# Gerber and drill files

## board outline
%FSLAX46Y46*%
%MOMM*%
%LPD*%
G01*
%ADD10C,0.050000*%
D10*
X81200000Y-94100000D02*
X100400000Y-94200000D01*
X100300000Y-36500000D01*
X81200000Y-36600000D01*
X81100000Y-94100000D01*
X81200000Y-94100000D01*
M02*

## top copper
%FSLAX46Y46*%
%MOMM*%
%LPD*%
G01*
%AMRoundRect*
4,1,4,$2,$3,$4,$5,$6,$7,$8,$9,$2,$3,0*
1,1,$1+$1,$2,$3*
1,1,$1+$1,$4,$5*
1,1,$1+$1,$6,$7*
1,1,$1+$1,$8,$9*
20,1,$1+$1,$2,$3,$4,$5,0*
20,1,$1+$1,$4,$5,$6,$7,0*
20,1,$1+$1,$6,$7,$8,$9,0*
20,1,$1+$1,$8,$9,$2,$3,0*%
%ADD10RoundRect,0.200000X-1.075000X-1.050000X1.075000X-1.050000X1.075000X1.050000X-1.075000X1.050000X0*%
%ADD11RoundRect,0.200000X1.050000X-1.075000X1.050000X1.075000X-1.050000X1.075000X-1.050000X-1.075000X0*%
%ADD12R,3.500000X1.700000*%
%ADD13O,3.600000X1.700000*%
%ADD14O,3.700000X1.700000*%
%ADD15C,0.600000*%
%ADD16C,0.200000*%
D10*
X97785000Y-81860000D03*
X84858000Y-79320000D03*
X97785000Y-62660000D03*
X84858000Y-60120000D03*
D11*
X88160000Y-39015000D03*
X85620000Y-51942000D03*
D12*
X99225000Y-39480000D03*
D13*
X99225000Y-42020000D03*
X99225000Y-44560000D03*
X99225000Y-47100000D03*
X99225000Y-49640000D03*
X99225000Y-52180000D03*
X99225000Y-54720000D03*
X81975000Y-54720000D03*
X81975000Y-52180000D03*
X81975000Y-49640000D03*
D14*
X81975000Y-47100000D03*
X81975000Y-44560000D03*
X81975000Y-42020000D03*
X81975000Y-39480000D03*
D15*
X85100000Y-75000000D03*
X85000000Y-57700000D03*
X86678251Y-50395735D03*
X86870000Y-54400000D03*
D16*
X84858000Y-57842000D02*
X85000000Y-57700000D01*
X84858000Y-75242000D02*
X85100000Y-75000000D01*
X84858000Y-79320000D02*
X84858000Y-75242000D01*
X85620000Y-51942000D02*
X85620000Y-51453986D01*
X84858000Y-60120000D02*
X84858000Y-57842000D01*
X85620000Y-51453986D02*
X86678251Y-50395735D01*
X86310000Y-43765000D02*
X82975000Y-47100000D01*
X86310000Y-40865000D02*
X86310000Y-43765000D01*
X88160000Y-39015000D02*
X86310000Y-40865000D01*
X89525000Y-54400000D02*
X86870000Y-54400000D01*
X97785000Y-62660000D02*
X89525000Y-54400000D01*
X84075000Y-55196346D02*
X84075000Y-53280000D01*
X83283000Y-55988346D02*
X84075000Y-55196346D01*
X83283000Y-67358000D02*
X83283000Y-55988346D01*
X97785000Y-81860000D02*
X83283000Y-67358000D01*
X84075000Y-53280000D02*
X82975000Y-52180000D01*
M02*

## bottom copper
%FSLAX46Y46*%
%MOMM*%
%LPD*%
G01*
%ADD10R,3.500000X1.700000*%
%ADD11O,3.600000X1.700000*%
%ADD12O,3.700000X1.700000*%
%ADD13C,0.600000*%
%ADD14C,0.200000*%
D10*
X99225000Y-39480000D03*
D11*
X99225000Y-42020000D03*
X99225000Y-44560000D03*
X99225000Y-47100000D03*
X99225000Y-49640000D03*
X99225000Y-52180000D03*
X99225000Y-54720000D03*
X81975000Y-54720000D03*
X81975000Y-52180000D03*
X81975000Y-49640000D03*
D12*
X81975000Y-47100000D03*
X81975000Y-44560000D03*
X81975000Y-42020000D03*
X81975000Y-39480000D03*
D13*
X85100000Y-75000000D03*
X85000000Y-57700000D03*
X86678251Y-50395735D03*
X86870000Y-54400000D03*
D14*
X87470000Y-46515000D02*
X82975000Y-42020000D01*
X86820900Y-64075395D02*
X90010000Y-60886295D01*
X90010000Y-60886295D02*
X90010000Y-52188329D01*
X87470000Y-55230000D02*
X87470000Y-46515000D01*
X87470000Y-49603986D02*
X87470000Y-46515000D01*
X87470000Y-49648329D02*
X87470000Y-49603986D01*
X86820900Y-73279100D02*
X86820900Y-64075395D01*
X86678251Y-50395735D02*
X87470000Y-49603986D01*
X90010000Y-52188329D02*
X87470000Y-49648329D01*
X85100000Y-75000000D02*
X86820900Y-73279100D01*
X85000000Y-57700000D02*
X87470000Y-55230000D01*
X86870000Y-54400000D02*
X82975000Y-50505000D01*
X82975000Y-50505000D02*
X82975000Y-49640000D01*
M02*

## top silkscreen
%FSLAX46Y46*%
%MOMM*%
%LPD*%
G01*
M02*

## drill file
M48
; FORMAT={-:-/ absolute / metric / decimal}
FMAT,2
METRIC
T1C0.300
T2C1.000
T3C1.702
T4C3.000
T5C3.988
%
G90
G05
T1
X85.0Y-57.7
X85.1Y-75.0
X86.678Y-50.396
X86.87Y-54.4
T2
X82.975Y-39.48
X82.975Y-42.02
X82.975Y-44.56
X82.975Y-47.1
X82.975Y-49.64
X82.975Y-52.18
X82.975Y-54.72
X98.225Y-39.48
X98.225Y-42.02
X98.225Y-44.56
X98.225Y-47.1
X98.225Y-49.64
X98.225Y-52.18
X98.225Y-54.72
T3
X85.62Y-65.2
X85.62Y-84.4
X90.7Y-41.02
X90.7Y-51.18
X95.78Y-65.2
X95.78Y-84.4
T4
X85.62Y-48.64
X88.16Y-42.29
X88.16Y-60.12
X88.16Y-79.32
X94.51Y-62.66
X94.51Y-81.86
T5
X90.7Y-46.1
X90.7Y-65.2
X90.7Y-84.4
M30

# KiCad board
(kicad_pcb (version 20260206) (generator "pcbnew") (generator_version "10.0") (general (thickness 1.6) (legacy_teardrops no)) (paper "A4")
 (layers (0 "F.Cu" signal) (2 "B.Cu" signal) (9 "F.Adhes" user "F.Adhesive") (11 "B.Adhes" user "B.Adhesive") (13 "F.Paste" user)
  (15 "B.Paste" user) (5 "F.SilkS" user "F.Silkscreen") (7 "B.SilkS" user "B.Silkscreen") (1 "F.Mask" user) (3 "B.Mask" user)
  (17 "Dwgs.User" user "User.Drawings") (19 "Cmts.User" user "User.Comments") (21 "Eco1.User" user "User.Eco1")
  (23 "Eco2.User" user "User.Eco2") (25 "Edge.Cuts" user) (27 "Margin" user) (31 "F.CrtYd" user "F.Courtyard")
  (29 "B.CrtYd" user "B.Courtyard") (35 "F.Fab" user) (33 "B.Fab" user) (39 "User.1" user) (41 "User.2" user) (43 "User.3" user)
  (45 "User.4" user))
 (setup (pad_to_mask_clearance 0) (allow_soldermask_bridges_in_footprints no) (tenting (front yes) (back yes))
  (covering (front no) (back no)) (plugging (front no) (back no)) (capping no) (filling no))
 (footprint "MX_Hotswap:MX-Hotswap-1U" (layer "F.Cu") (at 90.7 84.4)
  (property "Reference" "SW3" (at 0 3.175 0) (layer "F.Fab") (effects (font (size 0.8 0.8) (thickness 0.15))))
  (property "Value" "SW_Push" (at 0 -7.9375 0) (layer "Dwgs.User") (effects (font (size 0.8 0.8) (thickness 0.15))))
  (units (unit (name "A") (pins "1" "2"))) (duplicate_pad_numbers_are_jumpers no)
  (pad "" np_thru_hole circle (at -5.08 0 311.901) (size 1.7018 1.7018) (drill 1.7018) (layers "*.Cu" "*.Mask"))
  (pad "" np_thru_hole circle (at -2.54 -5.08) (size 3 3) (drill 3) (layers "*.Cu" "*.Mask"))
  (pad "" np_thru_hole circle (at 0 0) (size 3.9878 3.9878) (drill 3.9878) (layers "*.Cu" "*.Mask"))
  (pad "" np_thru_hole circle (at 3.81 -2.54) (size 3 3) (drill 3) (layers "*.Cu" "*.Mask"))
  (pad "" np_thru_hole circle (at 5.08 0 311.901) (size 1.7018 1.7018) (drill 1.7018) (layers "*.Cu" "*.Mask"))
  (pad "1" smd roundrect (at 7.085 -2.54) (size 2.55 2.5) (layers "F.Cu" "F.Mask" "F.Paste") (roundrect_rratio 0.08)
   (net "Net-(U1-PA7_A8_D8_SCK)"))
  (pad "2" smd roundrect (at -5.842 -5.08) (size 2.55 2.5) (layers "F.Cu" "F.Mask" "F.Paste") (roundrect_rratio 0.08) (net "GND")))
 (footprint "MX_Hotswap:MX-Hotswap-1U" (layer "F.Cu") (at 90.7 65.2)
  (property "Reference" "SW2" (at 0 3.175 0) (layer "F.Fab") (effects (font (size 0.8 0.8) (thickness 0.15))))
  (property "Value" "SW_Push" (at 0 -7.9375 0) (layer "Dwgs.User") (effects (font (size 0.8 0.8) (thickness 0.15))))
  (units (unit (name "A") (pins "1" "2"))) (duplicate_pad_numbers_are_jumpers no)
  (pad "" np_thru_hole circle (at -5.08 0 311.901) (size 1.7018 1.7018) (drill 1.7018) (layers "*.Cu" "*.Mask"))
  (pad "" np_thru_hole circle (at -2.54 -5.08) (size 3 3) (drill 3) (layers "*.Cu" "*.Mask"))
  (pad "" np_thru_hole circle (at 0 0) (size 3.9878 3.9878) (drill 3.9878) (layers "*.Cu" "*.Mask"))
  (pad "" np_thru_hole circle (at 3.81 -2.54) (size 3 3) (drill 3) (layers "*.Cu" "*.Mask"))
  (pad "" np_thru_hole circle (at 5.08 0 311.901) (size 1.7018 1.7018) (drill 1.7018) (layers "*.Cu" "*.Mask"))
  (pad "1" smd roundrect (at 7.085 -2.54) (size 2.55 2.5) (layers "F.Cu" "F.Mask" "F.Paste") (roundrect_rratio 0.08)
   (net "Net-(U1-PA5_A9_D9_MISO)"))
  (pad "2" smd roundrect (at -5.842 -5.08) (size 2.55 2.5) (layers "F.Cu" "F.Mask" "F.Paste") (roundrect_rratio 0.08) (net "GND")))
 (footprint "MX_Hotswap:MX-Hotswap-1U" (layer "F.Cu") (at 90.7 46.1 90)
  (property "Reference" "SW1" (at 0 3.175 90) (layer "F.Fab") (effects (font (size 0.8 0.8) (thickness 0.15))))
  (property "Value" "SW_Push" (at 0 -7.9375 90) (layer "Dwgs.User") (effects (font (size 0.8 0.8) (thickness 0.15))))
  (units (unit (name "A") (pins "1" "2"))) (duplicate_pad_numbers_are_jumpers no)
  (pad "" np_thru_hole circle (at -5.08 0 41.901) (size 1.7018 1.7018) (drill 1.7018) (layers "*.Cu" "*.Mask"))
  (pad "" np_thru_hole circle (at -2.54 -5.08 90) (size 3 3) (drill 3) (layers "*.Cu" "*.Mask"))
  (pad "" np_thru_hole circle (at 0 0 90) (size 3.9878 3.9878) (drill 3.9878) (layers "*.Cu" "*.Mask"))
  (pad "" np_thru_hole circle (at 3.81 -2.54 90) (size 3 3) (drill 3) (layers "*.Cu" "*.Mask"))
  (pad "" np_thru_hole circle (at 5.08 0 41.901) (size 1.7018 1.7018) (drill 1.7018) (layers "*.Cu" "*.Mask"))
  (pad "1" smd roundrect (at 7.085 -2.54 90) (size 2.55 2.5) (layers "F.Cu" "F.Mask" "F.Paste") (roundrect_rratio 0.08)
   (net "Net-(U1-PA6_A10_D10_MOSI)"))
  (pad "2" smd roundrect (at -5.842 -5.08 90) (size 2.55 2.5) (layers "F.Cu" "F.Mask" "F.Paste") (roundrect_rratio 0.08) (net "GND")))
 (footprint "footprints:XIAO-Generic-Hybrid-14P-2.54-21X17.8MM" (layer "B.Cu") (at 90.6 47.1 180)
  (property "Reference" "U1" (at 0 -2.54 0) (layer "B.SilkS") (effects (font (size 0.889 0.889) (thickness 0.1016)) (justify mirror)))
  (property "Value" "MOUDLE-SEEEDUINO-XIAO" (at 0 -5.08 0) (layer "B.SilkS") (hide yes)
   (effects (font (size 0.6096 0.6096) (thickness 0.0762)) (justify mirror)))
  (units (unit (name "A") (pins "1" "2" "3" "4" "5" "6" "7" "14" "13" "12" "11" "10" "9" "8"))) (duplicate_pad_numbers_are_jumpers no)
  (pad "1" thru_hole rect (at -7.625 7.62 180) (size 3.5 1.7) (drill 1 (offset -1 0)) (layers "*.Cu" "*.Mask") (remove_unused_layers no)
   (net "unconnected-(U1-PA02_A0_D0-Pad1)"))
  (pad "2" thru_hole oval (at -7.625 5.08 180) (size 3.6 1.7) (drill 1 (offset -1 0)) (layers "*.Cu" "*.Mask") (remove_unused_layers no)
   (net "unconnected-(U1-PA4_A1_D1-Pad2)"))
  (pad "3" thru_hole oval (at -7.625 2.54 180) (size 3.6 1.7) (drill 1 (offset -1 0)) (layers "*.Cu" "*.Mask") (remove_unused_layers no)
   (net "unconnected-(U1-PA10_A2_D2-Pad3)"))
  (pad "4" thru_hole oval (at -7.625 0 180) (size 3.6 1.7) (drill 1 (offset -1 0)) (layers "*.Cu" "*.Mask") (remove_unused_layers no)
   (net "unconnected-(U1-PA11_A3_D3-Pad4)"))
  (pad "5" thru_hole oval (at -7.625 -2.54 180) (size 3.6 1.7) (drill 1 (offset -1 0)) (layers "*.Cu" "*.Mask") (remove_unused_layers no)
   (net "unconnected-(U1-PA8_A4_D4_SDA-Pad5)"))
  (pad "6" thru_hole oval (at -7.625 -5.08) (size 3.6 1.7) (drill 1 (offset 1 0)) (layers "*.Cu" "*.Mask") (remove_unused_layers no)
   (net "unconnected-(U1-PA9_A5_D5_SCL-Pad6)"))
  (pad "7" thru_hole oval (at -7.625 -7.62 180) (size 3.6 1.7) (drill 1 (offset -1 0)) (layers "*.Cu" "*.Mask") (remove_unused_layers no)
   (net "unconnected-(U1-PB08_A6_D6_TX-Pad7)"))
  (pad "8" thru_hole oval (at 7.625 -7.62 180) (size 3.6 1.7) (drill 1 (offset 1 0)) (layers "*.Cu" "*.Mask") (remove_unused_layers no)
   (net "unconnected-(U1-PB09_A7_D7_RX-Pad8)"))
  (pad "9" thru_hole oval (at 7.625 -5.08 180) (size 3.6 1.7) (drill 1 (offset 1 0)) (layers "*.Cu" "*.Mask") (remove_unused_layers no)
   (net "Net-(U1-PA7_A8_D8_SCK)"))
  (pad "10" thru_hole oval (at 7.625 -2.54 180) (size 3.6 1.7) (drill 1 (offset 1 0)) (layers "*.Cu" "*.Mask") (remove_unused_layers no)
   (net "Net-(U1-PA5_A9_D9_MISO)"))
  (pad "11" thru_hole oval (at 7.625 0 180) (size 3.7 1.7) (drill 1 (offset 1 0)) (layers "*.Cu" "*.Mask") (remove_unused_layers no)
   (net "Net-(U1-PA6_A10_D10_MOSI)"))
  (pad "12" thru_hole oval (at 7.625 2.54 180) (size 3.7 1.7) (drill 1 (offset 1 0)) (layers "*.Cu" "*.Mask") (remove_unused_layers no)
   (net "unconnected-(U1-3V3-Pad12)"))
  (pad "13" thru_hole oval (at 7.625 5.08 180) (size 3.7 1.7) (drill 1 (offset 1 0)) (layers "*.Cu" "*.Mask") (remove_unused_layers no)
   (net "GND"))
  (pad "14" thru_hole oval (at 7.625 7.62 180) (size 3.7 1.7) (drill 1 (offset 1 0)) (layers "*.Cu" "*.Mask") (remove_unused_layers no)
   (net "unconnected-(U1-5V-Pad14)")))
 (gr_poly
  (pts (xy 81.2 94.1) (xy 100.4 94.2) (xy 100.3 36.5) (xy 81.2 36.6) (xy 81.1 94.1)) (stroke (width 0.05) (type solid)) (fill no)
  (layer "Edge.Cuts"))
 (segment (start 84.858 57.842) (end 85 57.7) (width 0.2) (layer "F.Cu") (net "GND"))
 (segment (start 84.858 75.242) (end 85.1 75) (width 0.2) (layer "F.Cu") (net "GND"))
 (segment (start 84.858 79.32) (end 84.858 75.242) (width 0.2) (layer "F.Cu") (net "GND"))
 (segment (start 85.62 51.942) (end 85.62 51.453986) (width 0.2) (layer "F.Cu") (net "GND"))
 (segment (start 84.858 60.12) (end 84.858 57.842) (width 0.2) (layer "F.Cu") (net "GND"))
 (segment (start 85.62 51.453986) (end 86.678251 50.395735) (width 0.2) (layer "F.Cu") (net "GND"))
 (via (at 85.1 75) (size 0.6) (drill 0.3) (layers "F.Cu" "B.Cu") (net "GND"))
 (via (at 85 57.7) (size 0.6) (drill 0.3) (layers "F.Cu" "B.Cu") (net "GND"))
 (via (at 86.678251 50.395735) (size 0.6) (drill 0.3) (layers "F.Cu" "B.Cu") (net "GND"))
 (segment (start 87.47 46.515) (end 82.975 42.02) (width 0.2) (layer "B.Cu") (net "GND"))
 (segment (start 86.8209 64.075395) (end 90.01 60.886295) (width 0.2) (layer "B.Cu") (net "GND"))
 (segment (start 90.01 60.886295) (end 90.01 52.188329) (width 0.2) (layer "B.Cu") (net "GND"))
 (segment (start 87.47 55.23) (end 87.47 46.515) (width 0.2) (layer "B.Cu") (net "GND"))
 (segment (start 87.47 49.603986) (end 87.47 46.515) (width 0.2) (layer "B.Cu") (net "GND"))
 (segment (start 87.47 49.648329) (end 87.47 49.603986) (width 0.2) (layer "B.Cu") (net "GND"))
 (segment (start 86.8209 73.2791) (end 86.8209 64.075395) (width 0.2) (layer "B.Cu") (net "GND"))
 (segment (start 86.678251 50.395735) (end 87.47 49.603986) (width 0.2) (layer "B.Cu") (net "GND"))
 (segment (start 90.01 52.188329) (end 87.47 49.648329) (width 0.2) (layer "B.Cu") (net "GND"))
 (segment (start 85.1 75) (end 86.8209 73.2791) (width 0.2) (layer "B.Cu") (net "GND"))
 (segment (start 85 57.7) (end 87.47 55.23) (width 0.2) (layer "B.Cu") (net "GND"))
 (segment (start 86.31 43.765) (end 82.975 47.1) (width 0.2) (layer "F.Cu") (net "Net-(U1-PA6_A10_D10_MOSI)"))
 (segment (start 86.31 40.865) (end 86.31 43.765) (width 0.2) (layer "F.Cu") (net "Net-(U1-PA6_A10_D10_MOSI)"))
 (segment (start 88.16 39.015) (end 86.31 40.865) (width 0.2) (layer "F.Cu") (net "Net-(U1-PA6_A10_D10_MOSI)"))
 (segment (start 89.525 54.4) (end 86.87 54.4) (width 0.2) (layer "F.Cu") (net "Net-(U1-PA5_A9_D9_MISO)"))
 (segment (start 97.785 62.66) (end 89.525 54.4) (width 0.2) (layer "F.Cu") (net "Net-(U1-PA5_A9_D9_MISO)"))
 (via (at 86.87 54.4) (size 0.6) (drill 0.3) (layers "F.Cu" "B.Cu") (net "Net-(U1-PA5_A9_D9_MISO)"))
 (segment (start 86.87 54.4) (end 82.975 50.505) (width 0.2) (layer "B.Cu") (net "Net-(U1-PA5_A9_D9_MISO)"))
 (segment (start 82.975 50.505) (end 82.975 49.64) (width 0.2) (layer "B.Cu") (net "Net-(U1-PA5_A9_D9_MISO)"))
 (segment (start 84.075 55.196346) (end 84.075 53.28) (width 0.2) (layer "F.Cu") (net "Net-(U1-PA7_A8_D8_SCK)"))
 (segment (start 83.283 55.988346) (end 84.075 55.196346) (width 0.2) (layer "F.Cu") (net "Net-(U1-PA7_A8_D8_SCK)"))
 (segment (start 83.283 67.358) (end 83.283 55.988346) (width 0.2) (layer "F.Cu") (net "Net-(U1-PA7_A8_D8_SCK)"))
 (segment (start 97.785 81.86) (end 83.283 67.358) (width 0.2) (layer "F.Cu") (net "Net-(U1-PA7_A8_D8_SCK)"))
 (segment (start 84.075 53.28) (end 82.975 52.18) (width 0.2) (layer "F.Cu") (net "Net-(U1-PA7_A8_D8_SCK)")))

